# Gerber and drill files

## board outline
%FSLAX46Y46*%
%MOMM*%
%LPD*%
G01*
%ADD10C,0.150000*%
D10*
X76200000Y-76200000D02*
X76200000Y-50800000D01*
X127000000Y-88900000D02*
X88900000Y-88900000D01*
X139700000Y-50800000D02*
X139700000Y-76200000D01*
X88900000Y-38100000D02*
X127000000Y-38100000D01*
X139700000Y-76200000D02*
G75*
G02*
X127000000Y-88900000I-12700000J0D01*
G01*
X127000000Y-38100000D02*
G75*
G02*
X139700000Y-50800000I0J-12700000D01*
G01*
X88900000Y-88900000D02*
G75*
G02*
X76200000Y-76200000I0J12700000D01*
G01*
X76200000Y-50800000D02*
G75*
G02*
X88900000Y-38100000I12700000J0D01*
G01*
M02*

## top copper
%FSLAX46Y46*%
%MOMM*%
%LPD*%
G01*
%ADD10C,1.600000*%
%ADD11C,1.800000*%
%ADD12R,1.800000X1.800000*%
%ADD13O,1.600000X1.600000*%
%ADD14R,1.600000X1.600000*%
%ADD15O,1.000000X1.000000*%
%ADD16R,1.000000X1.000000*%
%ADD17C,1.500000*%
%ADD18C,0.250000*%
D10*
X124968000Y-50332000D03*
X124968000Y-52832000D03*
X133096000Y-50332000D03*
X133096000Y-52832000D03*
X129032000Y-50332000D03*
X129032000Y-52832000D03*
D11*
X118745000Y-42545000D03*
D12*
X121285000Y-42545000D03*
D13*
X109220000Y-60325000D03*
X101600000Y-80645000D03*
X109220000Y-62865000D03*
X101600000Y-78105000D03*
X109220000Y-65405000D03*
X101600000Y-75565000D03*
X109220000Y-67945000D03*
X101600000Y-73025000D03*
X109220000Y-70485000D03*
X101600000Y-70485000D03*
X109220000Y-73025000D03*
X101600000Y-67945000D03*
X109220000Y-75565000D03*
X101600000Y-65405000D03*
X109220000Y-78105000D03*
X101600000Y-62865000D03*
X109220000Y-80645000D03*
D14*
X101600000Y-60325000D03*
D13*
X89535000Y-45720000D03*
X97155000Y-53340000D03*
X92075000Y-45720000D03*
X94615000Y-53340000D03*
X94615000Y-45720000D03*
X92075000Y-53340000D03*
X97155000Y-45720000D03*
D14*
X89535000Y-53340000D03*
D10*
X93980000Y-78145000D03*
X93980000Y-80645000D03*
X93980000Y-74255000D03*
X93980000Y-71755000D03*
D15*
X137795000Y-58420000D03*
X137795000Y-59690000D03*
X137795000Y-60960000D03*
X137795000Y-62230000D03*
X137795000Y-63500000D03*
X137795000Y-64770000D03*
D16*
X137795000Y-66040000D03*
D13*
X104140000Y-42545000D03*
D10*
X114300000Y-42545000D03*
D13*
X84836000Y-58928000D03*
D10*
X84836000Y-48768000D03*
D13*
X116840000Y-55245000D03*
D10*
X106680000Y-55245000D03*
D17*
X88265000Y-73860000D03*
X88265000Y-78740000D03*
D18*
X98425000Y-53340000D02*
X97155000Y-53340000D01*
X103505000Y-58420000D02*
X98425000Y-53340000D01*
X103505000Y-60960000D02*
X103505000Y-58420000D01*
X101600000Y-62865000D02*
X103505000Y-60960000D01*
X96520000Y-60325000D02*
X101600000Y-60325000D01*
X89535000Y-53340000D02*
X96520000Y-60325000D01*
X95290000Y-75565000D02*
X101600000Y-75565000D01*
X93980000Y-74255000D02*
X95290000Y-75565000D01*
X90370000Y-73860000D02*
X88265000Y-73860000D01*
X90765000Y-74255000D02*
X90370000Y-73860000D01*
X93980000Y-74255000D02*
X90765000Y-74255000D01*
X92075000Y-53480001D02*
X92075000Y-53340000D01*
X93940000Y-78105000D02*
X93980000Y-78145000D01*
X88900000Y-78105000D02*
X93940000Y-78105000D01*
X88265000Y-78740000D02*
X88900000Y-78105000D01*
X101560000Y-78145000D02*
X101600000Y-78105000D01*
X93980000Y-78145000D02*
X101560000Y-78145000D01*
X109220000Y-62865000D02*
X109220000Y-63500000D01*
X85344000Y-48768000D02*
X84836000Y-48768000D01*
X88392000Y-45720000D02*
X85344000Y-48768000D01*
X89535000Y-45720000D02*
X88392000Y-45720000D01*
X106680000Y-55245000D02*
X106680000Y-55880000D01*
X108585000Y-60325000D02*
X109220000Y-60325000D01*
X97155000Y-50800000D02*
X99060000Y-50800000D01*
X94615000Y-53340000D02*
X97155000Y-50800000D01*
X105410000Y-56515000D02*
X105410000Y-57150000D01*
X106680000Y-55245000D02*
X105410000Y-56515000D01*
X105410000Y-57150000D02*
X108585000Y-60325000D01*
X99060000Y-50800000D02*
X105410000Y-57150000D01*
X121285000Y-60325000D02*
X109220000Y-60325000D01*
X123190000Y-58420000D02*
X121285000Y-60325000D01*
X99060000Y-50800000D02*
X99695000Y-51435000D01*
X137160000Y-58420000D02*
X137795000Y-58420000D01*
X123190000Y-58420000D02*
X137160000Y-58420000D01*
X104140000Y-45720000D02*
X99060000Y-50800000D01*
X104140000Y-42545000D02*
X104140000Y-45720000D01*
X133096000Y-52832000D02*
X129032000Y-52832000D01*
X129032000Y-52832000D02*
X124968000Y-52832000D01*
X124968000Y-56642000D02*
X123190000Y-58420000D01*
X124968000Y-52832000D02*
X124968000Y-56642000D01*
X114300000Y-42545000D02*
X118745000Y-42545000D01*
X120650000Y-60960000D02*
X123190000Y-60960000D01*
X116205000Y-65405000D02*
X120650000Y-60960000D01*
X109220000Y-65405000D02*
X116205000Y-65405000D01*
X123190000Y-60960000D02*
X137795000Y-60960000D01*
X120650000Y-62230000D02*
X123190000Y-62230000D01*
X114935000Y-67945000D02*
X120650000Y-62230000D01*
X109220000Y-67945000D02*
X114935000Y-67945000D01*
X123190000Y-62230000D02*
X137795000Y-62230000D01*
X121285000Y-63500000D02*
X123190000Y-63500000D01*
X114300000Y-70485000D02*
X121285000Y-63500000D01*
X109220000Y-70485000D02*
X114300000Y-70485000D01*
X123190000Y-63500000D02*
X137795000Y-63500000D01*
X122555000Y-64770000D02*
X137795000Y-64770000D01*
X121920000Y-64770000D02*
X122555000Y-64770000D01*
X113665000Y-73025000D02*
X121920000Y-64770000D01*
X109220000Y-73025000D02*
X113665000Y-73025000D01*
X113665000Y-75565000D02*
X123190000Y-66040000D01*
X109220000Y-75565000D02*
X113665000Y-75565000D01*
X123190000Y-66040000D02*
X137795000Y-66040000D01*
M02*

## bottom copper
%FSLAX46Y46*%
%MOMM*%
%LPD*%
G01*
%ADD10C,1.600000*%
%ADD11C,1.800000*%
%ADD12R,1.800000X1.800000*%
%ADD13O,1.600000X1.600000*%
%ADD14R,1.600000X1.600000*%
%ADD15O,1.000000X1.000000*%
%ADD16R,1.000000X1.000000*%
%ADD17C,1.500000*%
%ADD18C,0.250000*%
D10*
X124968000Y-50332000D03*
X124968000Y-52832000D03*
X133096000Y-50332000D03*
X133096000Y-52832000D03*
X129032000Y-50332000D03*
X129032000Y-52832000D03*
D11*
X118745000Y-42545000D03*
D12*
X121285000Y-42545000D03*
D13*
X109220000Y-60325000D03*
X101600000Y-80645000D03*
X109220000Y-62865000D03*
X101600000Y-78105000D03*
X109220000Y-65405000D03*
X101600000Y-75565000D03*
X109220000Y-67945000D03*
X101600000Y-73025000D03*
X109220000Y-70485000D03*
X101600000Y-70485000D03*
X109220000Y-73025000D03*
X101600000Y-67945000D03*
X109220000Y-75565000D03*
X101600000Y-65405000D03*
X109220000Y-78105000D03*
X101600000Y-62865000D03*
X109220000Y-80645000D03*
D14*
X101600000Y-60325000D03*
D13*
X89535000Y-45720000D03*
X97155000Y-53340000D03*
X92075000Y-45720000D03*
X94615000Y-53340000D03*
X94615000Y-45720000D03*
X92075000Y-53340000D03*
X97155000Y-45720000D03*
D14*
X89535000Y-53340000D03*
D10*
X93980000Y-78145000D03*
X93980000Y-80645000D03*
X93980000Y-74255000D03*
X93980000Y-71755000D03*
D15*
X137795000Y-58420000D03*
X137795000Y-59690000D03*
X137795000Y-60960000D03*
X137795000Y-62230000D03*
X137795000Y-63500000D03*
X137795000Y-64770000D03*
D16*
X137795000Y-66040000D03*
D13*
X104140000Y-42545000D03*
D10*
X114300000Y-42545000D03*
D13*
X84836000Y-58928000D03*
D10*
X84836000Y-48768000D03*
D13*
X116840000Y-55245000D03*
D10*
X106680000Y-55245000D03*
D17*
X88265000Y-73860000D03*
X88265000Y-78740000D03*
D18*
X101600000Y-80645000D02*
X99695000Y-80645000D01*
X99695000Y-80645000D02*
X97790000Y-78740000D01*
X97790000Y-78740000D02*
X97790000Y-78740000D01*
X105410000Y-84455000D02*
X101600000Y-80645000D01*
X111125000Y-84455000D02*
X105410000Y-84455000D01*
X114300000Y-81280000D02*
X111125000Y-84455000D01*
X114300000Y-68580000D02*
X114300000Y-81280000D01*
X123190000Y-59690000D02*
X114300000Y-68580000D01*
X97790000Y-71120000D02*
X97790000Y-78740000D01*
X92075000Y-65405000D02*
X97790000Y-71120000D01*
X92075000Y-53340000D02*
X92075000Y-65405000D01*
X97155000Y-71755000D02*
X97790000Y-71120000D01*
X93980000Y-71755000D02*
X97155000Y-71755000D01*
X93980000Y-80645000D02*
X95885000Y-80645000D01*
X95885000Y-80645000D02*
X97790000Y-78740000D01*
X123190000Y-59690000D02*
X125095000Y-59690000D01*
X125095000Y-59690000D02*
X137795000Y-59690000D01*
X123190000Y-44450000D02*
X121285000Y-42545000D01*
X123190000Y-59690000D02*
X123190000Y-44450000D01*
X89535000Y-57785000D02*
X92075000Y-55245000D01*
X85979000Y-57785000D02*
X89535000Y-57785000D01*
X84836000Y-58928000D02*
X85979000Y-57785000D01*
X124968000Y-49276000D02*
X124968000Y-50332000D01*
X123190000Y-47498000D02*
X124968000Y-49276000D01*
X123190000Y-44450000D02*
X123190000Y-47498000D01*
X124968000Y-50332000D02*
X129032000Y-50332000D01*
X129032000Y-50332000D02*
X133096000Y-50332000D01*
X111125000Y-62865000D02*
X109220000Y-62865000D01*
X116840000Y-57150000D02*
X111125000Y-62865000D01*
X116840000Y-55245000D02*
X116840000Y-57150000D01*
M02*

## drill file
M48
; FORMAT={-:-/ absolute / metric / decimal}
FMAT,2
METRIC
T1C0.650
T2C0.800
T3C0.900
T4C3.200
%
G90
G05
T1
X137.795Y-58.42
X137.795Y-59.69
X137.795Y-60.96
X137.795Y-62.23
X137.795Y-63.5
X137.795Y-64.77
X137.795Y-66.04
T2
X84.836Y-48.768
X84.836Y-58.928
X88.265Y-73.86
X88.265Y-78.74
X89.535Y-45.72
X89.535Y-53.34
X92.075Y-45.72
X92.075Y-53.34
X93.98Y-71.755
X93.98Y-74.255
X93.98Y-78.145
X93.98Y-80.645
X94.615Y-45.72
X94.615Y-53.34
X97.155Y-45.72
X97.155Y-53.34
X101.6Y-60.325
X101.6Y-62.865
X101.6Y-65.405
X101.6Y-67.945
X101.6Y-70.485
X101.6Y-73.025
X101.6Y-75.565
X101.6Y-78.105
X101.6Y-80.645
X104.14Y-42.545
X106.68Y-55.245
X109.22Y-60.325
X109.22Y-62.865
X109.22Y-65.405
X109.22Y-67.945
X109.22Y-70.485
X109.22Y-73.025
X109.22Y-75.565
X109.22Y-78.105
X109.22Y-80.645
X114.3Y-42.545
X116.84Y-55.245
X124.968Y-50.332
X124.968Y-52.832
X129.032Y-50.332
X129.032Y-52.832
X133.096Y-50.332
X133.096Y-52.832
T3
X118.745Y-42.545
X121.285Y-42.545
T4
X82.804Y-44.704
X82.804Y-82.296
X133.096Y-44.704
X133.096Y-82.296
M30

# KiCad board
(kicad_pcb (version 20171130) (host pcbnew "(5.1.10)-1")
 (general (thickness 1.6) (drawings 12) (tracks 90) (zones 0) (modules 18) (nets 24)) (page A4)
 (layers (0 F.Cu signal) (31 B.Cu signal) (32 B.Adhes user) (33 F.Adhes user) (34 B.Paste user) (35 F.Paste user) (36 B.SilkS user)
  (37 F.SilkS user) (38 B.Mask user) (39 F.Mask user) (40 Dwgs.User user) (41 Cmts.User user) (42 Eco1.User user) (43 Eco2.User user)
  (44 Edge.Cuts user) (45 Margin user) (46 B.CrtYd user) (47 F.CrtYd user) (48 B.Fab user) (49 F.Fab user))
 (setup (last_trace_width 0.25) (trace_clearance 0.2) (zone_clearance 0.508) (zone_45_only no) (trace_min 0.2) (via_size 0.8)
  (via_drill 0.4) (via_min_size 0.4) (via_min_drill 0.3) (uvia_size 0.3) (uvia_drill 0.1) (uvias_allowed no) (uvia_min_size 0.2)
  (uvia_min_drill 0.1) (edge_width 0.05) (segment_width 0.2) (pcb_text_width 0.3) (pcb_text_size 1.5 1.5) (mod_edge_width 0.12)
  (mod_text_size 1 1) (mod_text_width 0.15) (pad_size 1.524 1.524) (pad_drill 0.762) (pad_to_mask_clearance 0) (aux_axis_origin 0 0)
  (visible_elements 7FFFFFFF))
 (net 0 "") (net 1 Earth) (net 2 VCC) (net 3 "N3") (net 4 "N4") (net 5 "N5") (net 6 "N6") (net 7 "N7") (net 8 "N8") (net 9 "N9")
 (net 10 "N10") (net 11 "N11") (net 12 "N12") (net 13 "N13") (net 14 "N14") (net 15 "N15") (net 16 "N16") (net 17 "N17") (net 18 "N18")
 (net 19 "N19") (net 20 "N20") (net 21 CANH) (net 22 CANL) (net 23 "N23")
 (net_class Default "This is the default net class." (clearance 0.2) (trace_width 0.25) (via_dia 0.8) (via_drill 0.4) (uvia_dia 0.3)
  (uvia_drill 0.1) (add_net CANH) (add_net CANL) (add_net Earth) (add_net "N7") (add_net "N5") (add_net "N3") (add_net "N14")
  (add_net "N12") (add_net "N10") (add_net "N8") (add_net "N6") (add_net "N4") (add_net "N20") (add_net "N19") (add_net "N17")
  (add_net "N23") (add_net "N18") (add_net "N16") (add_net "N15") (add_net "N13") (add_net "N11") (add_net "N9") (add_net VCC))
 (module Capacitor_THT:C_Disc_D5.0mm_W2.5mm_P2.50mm (layer F.Cu) (at 124.968 52.832 90)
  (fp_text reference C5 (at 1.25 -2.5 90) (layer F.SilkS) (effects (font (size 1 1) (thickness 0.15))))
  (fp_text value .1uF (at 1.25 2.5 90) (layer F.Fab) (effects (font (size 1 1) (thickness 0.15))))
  (pad 2 thru_hole circle (at 2.5 0 90) (size 1.6 1.6) (drill 0.8) (layers *.Cu *.Mask) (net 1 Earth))
  (pad 1 thru_hole circle (at 0 0 90) (size 1.6 1.6) (drill 0.8) (layers *.Cu *.Mask) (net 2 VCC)))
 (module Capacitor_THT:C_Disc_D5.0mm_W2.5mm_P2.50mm (layer F.Cu) (at 133.096 52.832 90)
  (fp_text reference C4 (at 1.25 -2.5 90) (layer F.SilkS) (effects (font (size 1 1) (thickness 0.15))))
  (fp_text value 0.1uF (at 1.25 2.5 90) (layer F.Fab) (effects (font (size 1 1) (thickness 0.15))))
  (pad 2 thru_hole circle (at 2.5 0 90) (size 1.6 1.6) (drill 0.8) (layers *.Cu *.Mask) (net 1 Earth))
  (pad 1 thru_hole circle (at 0 0 90) (size 1.6 1.6) (drill 0.8) (layers *.Cu *.Mask) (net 2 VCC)))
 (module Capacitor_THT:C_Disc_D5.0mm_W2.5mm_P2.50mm (layer F.Cu) (at 129.032 52.832 90)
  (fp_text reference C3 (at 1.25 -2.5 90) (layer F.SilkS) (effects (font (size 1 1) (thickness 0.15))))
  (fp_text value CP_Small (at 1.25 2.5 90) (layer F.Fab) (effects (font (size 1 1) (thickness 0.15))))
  (pad 2 thru_hole circle (at 2.5 0 90) (size 1.6 1.6) (drill 0.8) (layers *.Cu *.Mask) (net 1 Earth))
  (pad 1 thru_hole circle (at 0 0 90) (size 1.6 1.6) (drill 0.8) (layers *.Cu *.Mask) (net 2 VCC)))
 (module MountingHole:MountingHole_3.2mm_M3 (layer F.Cu) (at 82.804 82.296)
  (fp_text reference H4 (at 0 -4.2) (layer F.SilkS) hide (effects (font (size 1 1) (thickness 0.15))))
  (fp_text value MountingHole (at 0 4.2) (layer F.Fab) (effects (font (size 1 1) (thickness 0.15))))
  (pad 1 np_thru_hole circle (at 0 0) (size 3.2 3.2) (drill 3.2) (layers *.Cu *.Mask)))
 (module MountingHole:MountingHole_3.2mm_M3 (layer F.Cu) (at 82.804 44.704)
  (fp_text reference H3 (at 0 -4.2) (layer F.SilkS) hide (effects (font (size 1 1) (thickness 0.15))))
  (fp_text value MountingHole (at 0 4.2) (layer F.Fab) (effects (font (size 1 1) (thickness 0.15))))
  (pad 1 np_thru_hole circle (at 0 0) (size 3.2 3.2) (drill 3.2) (layers *.Cu *.Mask)))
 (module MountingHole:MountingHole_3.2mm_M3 (layer F.Cu) (at 133.096 82.296)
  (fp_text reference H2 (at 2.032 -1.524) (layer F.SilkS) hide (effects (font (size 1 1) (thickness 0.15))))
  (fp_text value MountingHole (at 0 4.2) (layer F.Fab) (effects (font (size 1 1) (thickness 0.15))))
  (pad 1 np_thru_hole circle (at 0 0) (size 3.2 3.2) (drill 3.2) (layers *.Cu *.Mask)))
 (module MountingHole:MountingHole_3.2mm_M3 (layer F.Cu) (at 133.096 44.704)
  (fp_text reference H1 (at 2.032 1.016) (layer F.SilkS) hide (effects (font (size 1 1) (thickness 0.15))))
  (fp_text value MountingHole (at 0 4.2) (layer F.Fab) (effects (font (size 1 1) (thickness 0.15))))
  (pad 1 np_thru_hole circle (at 0 0) (size 3.2 3.2) (drill 3.2) (layers *.Cu *.Mask)))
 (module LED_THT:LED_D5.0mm (layer F.Cu) (at 121.285 42.545 180)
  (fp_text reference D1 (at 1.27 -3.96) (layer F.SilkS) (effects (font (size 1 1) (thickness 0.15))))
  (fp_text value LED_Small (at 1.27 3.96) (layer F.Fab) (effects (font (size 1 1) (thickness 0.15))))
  (pad 2 thru_hole circle (at 2.54 0 180) (size 1.8 1.8) (drill 0.9) (layers *.Cu *.Mask) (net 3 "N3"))
  (pad 1 thru_hole rect (at 0 0 180) (size 1.8 1.8) (drill 0.9) (layers *.Cu *.Mask) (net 1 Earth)))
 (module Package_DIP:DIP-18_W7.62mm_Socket (layer F.Cu) (at 101.6 60.325)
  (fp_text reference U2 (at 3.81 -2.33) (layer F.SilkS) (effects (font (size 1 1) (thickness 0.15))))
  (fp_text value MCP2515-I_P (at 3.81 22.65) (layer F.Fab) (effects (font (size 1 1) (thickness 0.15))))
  (pad 18 thru_hole oval (at 7.62 0) (size 1.6 1.6) (drill 0.8) (layers *.Cu *.Mask) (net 2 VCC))
  (pad 9 thru_hole oval (at 0 20.32) (size 1.6 1.6) (drill 0.8) (layers *.Cu *.Mask) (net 1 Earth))
  (pad 17 thru_hole oval (at 7.62 2.54) (size 1.6 1.6) (drill 0.8) (layers *.Cu *.Mask) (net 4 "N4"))
  (pad 8 thru_hole oval (at 0 17.78) (size 1.6 1.6) (drill 0.8) (layers *.Cu *.Mask) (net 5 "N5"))
  (pad 16 thru_hole oval (at 7.62 5.08) (size 1.6 1.6) (drill 0.8) (layers *.Cu *.Mask) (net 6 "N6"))
  (pad 7 thru_hole oval (at 0 15.24) (size 1.6 1.6) (drill 0.8) (layers *.Cu *.Mask) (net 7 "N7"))
  (pad 15 thru_hole oval (at 7.62 7.62) (size 1.6 1.6) (drill 0.8) (layers *.Cu *.Mask) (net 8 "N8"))
  (pad 6 thru_hole oval (at 0 12.7) (size 1.6 1.6) (drill 0.8) (layers *.Cu *.Mask) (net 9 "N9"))
  (pad 14 thru_hole oval (at 7.62 10.16) (size 1.6 1.6) (drill 0.8) (layers *.Cu *.Mask) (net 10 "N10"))
  (pad 5 thru_hole oval (at 0 10.16) (size 1.6 1.6) (drill 0.8) (layers *.Cu *.Mask) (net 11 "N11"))
  (pad 13 thru_hole oval (at 7.62 12.7) (size 1.6 1.6) (drill 0.8) (layers *.Cu *.Mask) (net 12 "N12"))
  (pad 4 thru_hole oval (at 0 7.62) (size 1.6 1.6) (drill 0.8) (layers *.Cu *.Mask) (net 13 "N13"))
  (pad 12 thru_hole oval (at 7.62 15.24) (size 1.6 1.6) (drill 0.8) (layers *.Cu *.Mask) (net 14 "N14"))
  (pad 3 thru_hole oval (at 0 5.08) (size 1.6 1.6) (drill 0.8) (layers *.Cu *.Mask) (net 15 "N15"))
  (pad 11 thru_hole oval (at 7.62 17.78) (size 1.6 1.6) (drill 0.8) (layers *.Cu *.Mask) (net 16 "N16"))
  (pad 2 thru_hole oval (at 0 2.54) (size 1.6 1.6) (drill 0.8) (layers *.Cu *.Mask) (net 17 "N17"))
  (pad 10 thru_hole oval (at 7.62 20.32) (size 1.6 1.6) (drill 0.8) (layers *.Cu *.Mask) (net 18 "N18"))
  (pad 1 thru_hole rect (at 0 0) (size 1.6 1.6) (drill 0.8) (layers *.Cu *.Mask) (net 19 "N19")))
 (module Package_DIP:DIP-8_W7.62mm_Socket (layer F.Cu) (at 89.535 53.34 90)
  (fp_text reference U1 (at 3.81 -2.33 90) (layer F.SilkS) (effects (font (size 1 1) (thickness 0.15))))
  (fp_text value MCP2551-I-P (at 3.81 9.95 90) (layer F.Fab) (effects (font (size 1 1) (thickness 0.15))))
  (pad 8 thru_hole oval (at 7.62 0 90) (size 1.6 1.6) (drill 0.8) (layers *.Cu *.Mask) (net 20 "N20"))
  (pad 4 thru_hole oval (at 0 7.62 90) (size 1.6 1.6) (drill 0.8) (layers *.Cu *.Mask) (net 17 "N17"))
  (pad 7 thru_hole oval (at 7.62 2.54 90) (size 1.6 1.6) (drill 0.8) (layers *.Cu *.Mask) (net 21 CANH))
  (pad 3 thru_hole oval (at 0 5.08 90) (size 1.6 1.6) (drill 0.8) (layers *.Cu *.Mask) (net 2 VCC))
  (pad 6 thru_hole oval (at 7.62 5.08 90) (size 1.6 1.6) (drill 0.8) (layers *.Cu *.Mask) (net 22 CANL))
  (pad 2 thru_hole oval (at 0 2.54 90) (size 1.6 1.6) (drill 0.8) (layers *.Cu *.Mask) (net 1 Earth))
  (pad 5 thru_hole oval (at 7.62 7.62 90) (size 1.6 1.6) (drill 0.8) (layers *.Cu *.Mask) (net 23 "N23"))
  (pad 1 thru_hole rect (at 0 0 90) (size 1.6 1.6) (drill 0.8) (layers *.Cu *.Mask) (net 19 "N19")))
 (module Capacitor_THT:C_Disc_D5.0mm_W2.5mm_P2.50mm (layer F.Cu) (at 93.98 80.645 90)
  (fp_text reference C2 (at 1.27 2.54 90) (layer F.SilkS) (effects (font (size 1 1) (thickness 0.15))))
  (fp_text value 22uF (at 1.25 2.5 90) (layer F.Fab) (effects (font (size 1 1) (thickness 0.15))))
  (pad 2 thru_hole circle (at 2.5 0 90) (size 1.6 1.6) (drill 0.8) (layers *.Cu *.Mask) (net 5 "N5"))
  (pad 1 thru_hole circle (at 0 0 90) (size 1.6 1.6) (drill 0.8) (layers *.Cu *.Mask) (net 1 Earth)))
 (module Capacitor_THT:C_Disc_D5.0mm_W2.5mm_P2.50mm (layer F.Cu) (at 93.98 71.755 270)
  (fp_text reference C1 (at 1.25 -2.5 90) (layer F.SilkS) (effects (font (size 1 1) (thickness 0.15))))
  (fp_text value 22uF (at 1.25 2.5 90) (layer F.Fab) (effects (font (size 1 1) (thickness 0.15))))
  (pad 2 thru_hole circle (at 2.5 0 270) (size 1.6 1.6) (drill 0.8) (layers *.Cu *.Mask) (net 7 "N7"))
  (pad 1 thru_hole circle (at 0 0 270) (size 1.6 1.6) (drill 0.8) (layers *.Cu *.Mask) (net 1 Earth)))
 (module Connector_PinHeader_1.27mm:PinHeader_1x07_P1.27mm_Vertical (layer F.Cu) (at 137.795 66.04 180)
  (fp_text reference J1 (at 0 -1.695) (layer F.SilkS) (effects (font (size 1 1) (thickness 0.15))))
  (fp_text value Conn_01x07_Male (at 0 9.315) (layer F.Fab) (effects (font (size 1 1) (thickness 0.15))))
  (pad 7 thru_hole oval (at 0 7.62 180) (size 1 1) (drill 0.65) (layers *.Cu *.Mask) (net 2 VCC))
  (pad 6 thru_hole oval (at 0 6.35 180) (size 1 1) (drill 0.65) (layers *.Cu *.Mask) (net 1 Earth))
  (pad 5 thru_hole oval (at 0 5.08 180) (size 1 1) (drill 0.65) (layers *.Cu *.Mask) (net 6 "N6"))
  (pad 4 thru_hole oval (at 0 3.81 180) (size 1 1) (drill 0.65) (layers *.Cu *.Mask) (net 8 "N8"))
  (pad 3 thru_hole oval (at 0 2.54 180) (size 1 1) (drill 0.65) (layers *.Cu *.Mask) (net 10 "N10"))
  (pad 2 thru_hole oval (at 0 1.27 180) (size 1 1) (drill 0.65) (layers *.Cu *.Mask) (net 12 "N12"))
  (pad 1 thru_hole rect (at 0 0 180) (size 1 1) (drill 0.65) (layers *.Cu *.Mask) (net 14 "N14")))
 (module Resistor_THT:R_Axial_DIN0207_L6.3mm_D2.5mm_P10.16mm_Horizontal (layer F.Cu) (at 114.3 42.545 180)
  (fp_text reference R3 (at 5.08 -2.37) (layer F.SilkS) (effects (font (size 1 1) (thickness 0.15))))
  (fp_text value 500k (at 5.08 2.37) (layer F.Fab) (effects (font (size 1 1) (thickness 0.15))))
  (pad 2 thru_hole oval (at 10.16 0 180) (size 1.6 1.6) (drill 0.8) (layers *.Cu *.Mask) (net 2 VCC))
  (pad 1 thru_hole circle (at 0 0 180) (size 1.6 1.6) (drill 0.8) (layers *.Cu *.Mask) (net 3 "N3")))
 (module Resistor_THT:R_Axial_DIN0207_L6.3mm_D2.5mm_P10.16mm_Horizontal (layer F.Cu) (at 84.836 48.768 270)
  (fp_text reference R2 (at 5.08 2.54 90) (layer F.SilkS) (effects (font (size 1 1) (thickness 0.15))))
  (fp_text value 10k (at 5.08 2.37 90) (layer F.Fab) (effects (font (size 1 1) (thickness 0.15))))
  (pad 2 thru_hole oval (at 10.16 0 270) (size 1.6 1.6) (drill 0.8) (layers *.Cu *.Mask) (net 1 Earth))
  (pad 1 thru_hole circle (at 0 0 270) (size 1.6 1.6) (drill 0.8) (layers *.Cu *.Mask) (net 20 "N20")))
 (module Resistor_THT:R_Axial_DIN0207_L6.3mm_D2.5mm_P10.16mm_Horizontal (layer F.Cu) (at 106.68 55.245)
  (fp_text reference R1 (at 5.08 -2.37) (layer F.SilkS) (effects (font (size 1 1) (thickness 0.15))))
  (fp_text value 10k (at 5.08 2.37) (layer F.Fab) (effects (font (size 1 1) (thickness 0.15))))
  (pad 2 thru_hole oval (at 10.16 0) (size 1.6 1.6) (drill 0.8) (layers *.Cu *.Mask) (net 4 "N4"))
  (pad 1 thru_hole circle (at 0 0) (size 1.6 1.6) (drill 0.8) (layers *.Cu *.Mask) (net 2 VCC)))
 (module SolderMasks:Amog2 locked (layer B.Cu) (at 107.95 62.23 90)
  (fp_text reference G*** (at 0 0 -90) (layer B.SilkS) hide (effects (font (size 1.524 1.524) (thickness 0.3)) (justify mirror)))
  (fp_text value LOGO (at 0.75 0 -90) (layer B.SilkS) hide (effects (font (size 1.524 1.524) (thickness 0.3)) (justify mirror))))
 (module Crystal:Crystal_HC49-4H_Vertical (layer F.Cu) (at 88.265 78.74 90)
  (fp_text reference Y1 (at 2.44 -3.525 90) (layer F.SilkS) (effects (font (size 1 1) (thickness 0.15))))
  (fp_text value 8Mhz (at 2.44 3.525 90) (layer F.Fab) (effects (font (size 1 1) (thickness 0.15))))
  (pad 2 thru_hole circle (at 4.88 0 90) (size 1.5 1.5) (drill 0.8) (layers *.Cu *.Mask) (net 7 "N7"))
  (pad 1 thru_hole circle (at 0 0 90) (size 1.5 1.5) (drill 0.8) (layers *.Cu *.Mask) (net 5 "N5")))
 (gr_line (start 76.2 76.2) (end 76.2 50.8) (layer Edge.Cuts) (width 0.15))
 (gr_line (start 127 88.9) (end 88.9 88.9) (layer Edge.Cuts) (width 0.15))
 (gr_line (start 139.7 50.8) (end 139.7 76.2) (layer Edge.Cuts) (width 0.15))
 (gr_line (start 88.9 38.1) (end 127 38.1) (layer Edge.Cuts) (width 0.15))
 (gr_arc (start 127 76.2) (end 127 88.9) (angle -90) (layer Edge.Cuts) (width 0.15))
 (gr_arc (start 127 50.8) (end 139.7 50.8) (angle -90) (layer Edge.Cuts) (width 0.15))
 (gr_arc (start 88.9 76.2) (end 76.2 76.2) (angle -90) (layer Edge.Cuts) (width 0.15))
 (gr_arc (start 88.9 50.8) (end 88.9 38.1) (angle -90) (layer Edge.Cuts) (width 0.15))
 (segment (start 98.425 53.34) (end 97.155 53.34) (width 0.25) (layer F.Cu) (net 17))
 (segment (start 103.505 58.42) (end 98.425 53.34) (width 0.25) (layer F.Cu) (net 17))
 (segment (start 103.505 60.96) (end 103.505 58.42) (width 0.25) (layer F.Cu) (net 17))
 (segment (start 101.6 62.865) (end 103.505 60.96) (width 0.25) (layer F.Cu) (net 17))
 (segment (start 96.52 60.325) (end 101.6 60.325) (width 0.25) (layer F.Cu) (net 19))
 (segment (start 89.535 53.34) (end 96.52 60.325) (width 0.25) (layer F.Cu) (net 19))
 (segment (start 95.29 75.565) (end 101.6 75.565) (width 0.25) (layer F.Cu) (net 7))
 (segment (start 93.98 74.255) (end 95.29 75.565) (width 0.25) (layer F.Cu) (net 7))
 (segment (start 90.37 73.86) (end 88.265 73.86) (width 0.25) (layer F.Cu) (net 7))
 (segment (start 90.765 74.255) (end 90.37 73.86) (width 0.25) (layer F.Cu) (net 7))
 (segment (start 93.98 74.255) (end 90.765 74.255) (width 0.25) (layer F.Cu) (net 7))
 (segment (start 101.6 80.645) (end 99.695 80.645) (width 0.25) (layer B.Cu) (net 1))
 (segment (start 99.695 80.645) (end 97.79 78.74) (width 0.25) (layer B.Cu) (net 1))
 (segment (start 97.79 78.74) (end 97.79 78.74) (width 0.25) (layer B.Cu) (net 1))
 (segment (start 92.075 53.480001) (end 92.075 53.34) (width 0.25) (layer F.Cu) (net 1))
 (segment (start 105.41 84.455) (end 101.6 80.645) (width 0.25) (layer B.Cu) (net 1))
 (segment (start 111.125 84.455) (end 105.41 84.455) (width 0.25) (layer B.Cu) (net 1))
 (segment (start 114.3 81.28) (end 111.125 84.455) (width 0.25) (layer B.Cu) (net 1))
 (segment (start 114.3 68.58) (end 114.3 81.28) (width 0.25) (layer B.Cu) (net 1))
 (segment (start 123.19 59.69) (end 114.3 68.58) (width 0.25) (layer B.Cu) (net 1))
 (segment (start 97.79 71.12) (end 97.79 78.74) (width 0.25) (layer B.Cu) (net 1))
 (segment (start 92.075 65.405) (end 97.79 71.12) (width 0.25) (layer B.Cu) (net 1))
 (segment (start 92.075 53.34) (end 92.075 65.405) (width 0.25) (layer B.Cu) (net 1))
 (segment (start 97.155 71.755) (end 97.79 71.12) (width 0.25) (layer B.Cu) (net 1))
 (segment (start 93.98 71.755) (end 97.155 71.755) (width 0.25) (layer B.Cu) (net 1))
 (segment (start 93.98 80.645) (end 95.885 80.645) (width 0.25) (layer B.Cu) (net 1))
 (segment (start 95.885 80.645) (end 97.79 78.74) (width 0.25) (layer B.Cu) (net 1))
 (segment (start 123.19 59.69) (end 125.095 59.69) (width 0.25) (layer B.Cu) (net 1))
 (segment (start 125.095 59.69) (end 137.795 59.69) (width 0.25) (layer B.Cu) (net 1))
 (segment (start 123.19 44.45) (end 121.285 42.545) (width 0.25) (layer B.Cu) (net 1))
 (segment (start 123.19 59.69) (end 123.19 44.45) (width 0.25) (layer B.Cu) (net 1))
 (segment (start 89.535 57.785) (end 92.075 55.245) (width 0.25) (layer B.Cu) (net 1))
 (segment (start 85.979 57.785) (end 89.535 57.785) (width 0.25) (layer B.Cu) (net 1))
 (segment (start 84.836 58.928) (end 85.979 57.785) (width 0.25) (layer B.Cu) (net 1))
 (segment (start 124.968 49.276) (end 124.968 50.332) (width 0.25) (layer B.Cu) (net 1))
 (segment (start 123.19 47.498) (end 124.968 49.276) (width 0.25) (layer B.Cu) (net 1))
 (segment (start 123.19 44.45) (end 123.19 47.498) (width 0.25) (layer B.Cu) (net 1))
 (segment (start 124.968 50.332) (end 129.032 50.332) (width 0.25) (layer B.Cu) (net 1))
 (segment (start 129.032 50.332) (end 133.096 50.332) (width 0.25) (layer B.Cu) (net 1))
 (segment (start 93.94 78.105) (end 93.98 78.145) (width 0.25) (layer F.Cu) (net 5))
 (segment (start 88.9 78.105) (end 93.94 78.105) (width 0.25) (layer F.Cu) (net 5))
 (segment (start 88.265 78.74) (end 88.9 78.105) (width 0.25) (layer F.Cu) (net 5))
 (segment (start 101.56 78.145) (end 101.6 78.105) (width 0.25) (layer F.Cu) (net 5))
 (segment (start 93.98 78.145) (end 101.56 78.145) (width 0.25) (layer F.Cu) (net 5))
 (segment (start 109.22 62.865) (end 109.22 63.5) (width 0.25) (layer F.Cu) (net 4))
 (segment (start 111.125 62.865) (end 109.22 62.865) (width 0.25) (layer B.Cu) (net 4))
 (segment (start 116.84 57.15) (end 111.125 62.865) (width 0.25) (layer B.Cu) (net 4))
 (segment (start 116.84 55.245) (end 116.84 57.15) (width 0.25) (layer B.Cu) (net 4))
 (segment (start 85.344 48.768) (end 84.836 48.768) (width 0.25) (layer F.Cu) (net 20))
 (segment (start 88.392 45.72) (end 85.344 48.768) (width 0.25) (layer F.Cu) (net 20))
 (segment (start 89.535 45.72) (end 88.392 45.72) (width 0.25) (layer F.Cu) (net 20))
 (segment (start 106.68 55.245) (end 106.68 55.88) (width 0.25) (layer F.Cu) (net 2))
 (segment (start 108.585 60.325) (end 109.22 60.325) (width 0.25) (layer F.Cu) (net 2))
 (segment (start 97.155 50.8) (end 99.06 50.8) (width 0.25) (layer F.Cu) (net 2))
 (segment (start 94.615 53.34) (end 97.155 50.8) (width 0.25) (layer F.Cu) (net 2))
 (segment (start 105.41 56.515) (end 105.41 57.15) (width 0.25) (layer F.Cu) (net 2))
 (segment (start 106.68 55.245) (end 105.41 56.515) (width 0.25) (layer F.Cu) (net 2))
 (segment (start 105.41 57.15) (end 108.585 60.325) (width 0.25) (layer F.Cu) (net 2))
 (segment (start 99.06 50.8) (end 105.41 57.15) (width 0.25) (layer F.Cu) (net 2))
 (segment (start 121.285 60.325) (end 109.22 60.325) (width 0.25) (layer F.Cu) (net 2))
 (segment (start 123.19 58.42) (end 121.285 60.325) (width 0.25) (layer F.Cu) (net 2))
 (segment (start 99.06 50.8) (end 99.695 51.435) (width 0.25) (layer F.Cu) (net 2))
 (segment (start 137.16 58.42) (end 137.795 58.42) (width 0.25) (layer F.Cu) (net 2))
 (segment (start 123.19 58.42) (end 137.16 58.42) (width 0.25) (layer F.Cu) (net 2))
 (segment (start 104.14 45.72) (end 99.06 50.8) (width 0.25) (layer F.Cu) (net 2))
 (segment (start 104.14 42.545) (end 104.14 45.72) (width 0.25) (layer F.Cu) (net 2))
 (segment (start 133.096 52.832) (end 129.032 52.832) (width 0.25) (layer F.Cu) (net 2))
 (segment (start 129.032 52.832) (end 124.968 52.832) (width 0.25) (layer F.Cu) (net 2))
 (segment (start 124.968 56.642) (end 123.19 58.42) (width 0.25) (layer F.Cu) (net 2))
 (segment (start 124.968 52.832) (end 124.968 56.642) (width 0.25) (layer F.Cu) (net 2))
 (segment (start 114.3 42.545) (end 118.745 42.545) (width 0.25) (layer F.Cu) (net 3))
 (segment (start 120.65 60.96) (end 123.19 60.96) (width 0.25) (layer F.Cu) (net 6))
 (segment (start 116.205 65.405) (end 120.65 60.96) (width 0.25) (layer F.Cu) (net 6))
 (segment (start 109.22 65.405) (end 116.205 65.405) (width 0.25) (layer F.Cu) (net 6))
 (segment (start 123.19 60.96) (end 137.795 60.96) (width 0.25) (layer F.Cu) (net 6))
 (segment (start 120.65 62.23) (end 123.19 62.23) (width 0.25) (layer F.Cu) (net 8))
 (segment (start 114.935 67.945) (end 120.65 62.23) (width 0.25) (layer F.Cu) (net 8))
 (segment (start 109.22 67.945) (end 114.935 67.945) (width 0.25) (layer F.Cu) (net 8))
 (segment (start 123.19 62.23) (end 137.795 62.23) (width 0.25) (layer F.Cu) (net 8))
 (segment (start 121.285 63.5) (end 123.19 63.5) (width 0.25) (layer F.Cu) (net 10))
 (segment (start 114.3 70.485) (end 121.285 63.5) (width 0.25) (layer F.Cu) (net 10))
 (segment (start 109.22 70.485) (end 114.3 70.485) (width 0.25) (layer F.Cu) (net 10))
 (segment (start 123.19 63.5) (end 137.795 63.5) (width 0.25) (layer F.Cu) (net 10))
 (segment (start 122.555 64.77) (end 137.795 64.77) (width 0.25) (layer F.Cu) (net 12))
 (segment (start 121.92 64.77) (end 122.555 64.77) (width 0.25) (layer F.Cu) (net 12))
 (segment (start 113.665 73.025) (end 121.92 64.77) (width 0.25) (layer F.Cu) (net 12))
 (segment (start 109.22 73.025) (end 113.665 73.025) (width 0.25) (layer F.Cu) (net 12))
 (segment (start 113.665 75.565) (end 123.19 66.04) (width 0.25) (layer F.Cu) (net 14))
 (segment (start 109.22 75.565) (end 113.665 75.565) (width 0.25) (layer F.Cu) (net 14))
 (segment (start 123.19 66.04) (end 137.795 66.04) (width 0.25) (layer F.Cu) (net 14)))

